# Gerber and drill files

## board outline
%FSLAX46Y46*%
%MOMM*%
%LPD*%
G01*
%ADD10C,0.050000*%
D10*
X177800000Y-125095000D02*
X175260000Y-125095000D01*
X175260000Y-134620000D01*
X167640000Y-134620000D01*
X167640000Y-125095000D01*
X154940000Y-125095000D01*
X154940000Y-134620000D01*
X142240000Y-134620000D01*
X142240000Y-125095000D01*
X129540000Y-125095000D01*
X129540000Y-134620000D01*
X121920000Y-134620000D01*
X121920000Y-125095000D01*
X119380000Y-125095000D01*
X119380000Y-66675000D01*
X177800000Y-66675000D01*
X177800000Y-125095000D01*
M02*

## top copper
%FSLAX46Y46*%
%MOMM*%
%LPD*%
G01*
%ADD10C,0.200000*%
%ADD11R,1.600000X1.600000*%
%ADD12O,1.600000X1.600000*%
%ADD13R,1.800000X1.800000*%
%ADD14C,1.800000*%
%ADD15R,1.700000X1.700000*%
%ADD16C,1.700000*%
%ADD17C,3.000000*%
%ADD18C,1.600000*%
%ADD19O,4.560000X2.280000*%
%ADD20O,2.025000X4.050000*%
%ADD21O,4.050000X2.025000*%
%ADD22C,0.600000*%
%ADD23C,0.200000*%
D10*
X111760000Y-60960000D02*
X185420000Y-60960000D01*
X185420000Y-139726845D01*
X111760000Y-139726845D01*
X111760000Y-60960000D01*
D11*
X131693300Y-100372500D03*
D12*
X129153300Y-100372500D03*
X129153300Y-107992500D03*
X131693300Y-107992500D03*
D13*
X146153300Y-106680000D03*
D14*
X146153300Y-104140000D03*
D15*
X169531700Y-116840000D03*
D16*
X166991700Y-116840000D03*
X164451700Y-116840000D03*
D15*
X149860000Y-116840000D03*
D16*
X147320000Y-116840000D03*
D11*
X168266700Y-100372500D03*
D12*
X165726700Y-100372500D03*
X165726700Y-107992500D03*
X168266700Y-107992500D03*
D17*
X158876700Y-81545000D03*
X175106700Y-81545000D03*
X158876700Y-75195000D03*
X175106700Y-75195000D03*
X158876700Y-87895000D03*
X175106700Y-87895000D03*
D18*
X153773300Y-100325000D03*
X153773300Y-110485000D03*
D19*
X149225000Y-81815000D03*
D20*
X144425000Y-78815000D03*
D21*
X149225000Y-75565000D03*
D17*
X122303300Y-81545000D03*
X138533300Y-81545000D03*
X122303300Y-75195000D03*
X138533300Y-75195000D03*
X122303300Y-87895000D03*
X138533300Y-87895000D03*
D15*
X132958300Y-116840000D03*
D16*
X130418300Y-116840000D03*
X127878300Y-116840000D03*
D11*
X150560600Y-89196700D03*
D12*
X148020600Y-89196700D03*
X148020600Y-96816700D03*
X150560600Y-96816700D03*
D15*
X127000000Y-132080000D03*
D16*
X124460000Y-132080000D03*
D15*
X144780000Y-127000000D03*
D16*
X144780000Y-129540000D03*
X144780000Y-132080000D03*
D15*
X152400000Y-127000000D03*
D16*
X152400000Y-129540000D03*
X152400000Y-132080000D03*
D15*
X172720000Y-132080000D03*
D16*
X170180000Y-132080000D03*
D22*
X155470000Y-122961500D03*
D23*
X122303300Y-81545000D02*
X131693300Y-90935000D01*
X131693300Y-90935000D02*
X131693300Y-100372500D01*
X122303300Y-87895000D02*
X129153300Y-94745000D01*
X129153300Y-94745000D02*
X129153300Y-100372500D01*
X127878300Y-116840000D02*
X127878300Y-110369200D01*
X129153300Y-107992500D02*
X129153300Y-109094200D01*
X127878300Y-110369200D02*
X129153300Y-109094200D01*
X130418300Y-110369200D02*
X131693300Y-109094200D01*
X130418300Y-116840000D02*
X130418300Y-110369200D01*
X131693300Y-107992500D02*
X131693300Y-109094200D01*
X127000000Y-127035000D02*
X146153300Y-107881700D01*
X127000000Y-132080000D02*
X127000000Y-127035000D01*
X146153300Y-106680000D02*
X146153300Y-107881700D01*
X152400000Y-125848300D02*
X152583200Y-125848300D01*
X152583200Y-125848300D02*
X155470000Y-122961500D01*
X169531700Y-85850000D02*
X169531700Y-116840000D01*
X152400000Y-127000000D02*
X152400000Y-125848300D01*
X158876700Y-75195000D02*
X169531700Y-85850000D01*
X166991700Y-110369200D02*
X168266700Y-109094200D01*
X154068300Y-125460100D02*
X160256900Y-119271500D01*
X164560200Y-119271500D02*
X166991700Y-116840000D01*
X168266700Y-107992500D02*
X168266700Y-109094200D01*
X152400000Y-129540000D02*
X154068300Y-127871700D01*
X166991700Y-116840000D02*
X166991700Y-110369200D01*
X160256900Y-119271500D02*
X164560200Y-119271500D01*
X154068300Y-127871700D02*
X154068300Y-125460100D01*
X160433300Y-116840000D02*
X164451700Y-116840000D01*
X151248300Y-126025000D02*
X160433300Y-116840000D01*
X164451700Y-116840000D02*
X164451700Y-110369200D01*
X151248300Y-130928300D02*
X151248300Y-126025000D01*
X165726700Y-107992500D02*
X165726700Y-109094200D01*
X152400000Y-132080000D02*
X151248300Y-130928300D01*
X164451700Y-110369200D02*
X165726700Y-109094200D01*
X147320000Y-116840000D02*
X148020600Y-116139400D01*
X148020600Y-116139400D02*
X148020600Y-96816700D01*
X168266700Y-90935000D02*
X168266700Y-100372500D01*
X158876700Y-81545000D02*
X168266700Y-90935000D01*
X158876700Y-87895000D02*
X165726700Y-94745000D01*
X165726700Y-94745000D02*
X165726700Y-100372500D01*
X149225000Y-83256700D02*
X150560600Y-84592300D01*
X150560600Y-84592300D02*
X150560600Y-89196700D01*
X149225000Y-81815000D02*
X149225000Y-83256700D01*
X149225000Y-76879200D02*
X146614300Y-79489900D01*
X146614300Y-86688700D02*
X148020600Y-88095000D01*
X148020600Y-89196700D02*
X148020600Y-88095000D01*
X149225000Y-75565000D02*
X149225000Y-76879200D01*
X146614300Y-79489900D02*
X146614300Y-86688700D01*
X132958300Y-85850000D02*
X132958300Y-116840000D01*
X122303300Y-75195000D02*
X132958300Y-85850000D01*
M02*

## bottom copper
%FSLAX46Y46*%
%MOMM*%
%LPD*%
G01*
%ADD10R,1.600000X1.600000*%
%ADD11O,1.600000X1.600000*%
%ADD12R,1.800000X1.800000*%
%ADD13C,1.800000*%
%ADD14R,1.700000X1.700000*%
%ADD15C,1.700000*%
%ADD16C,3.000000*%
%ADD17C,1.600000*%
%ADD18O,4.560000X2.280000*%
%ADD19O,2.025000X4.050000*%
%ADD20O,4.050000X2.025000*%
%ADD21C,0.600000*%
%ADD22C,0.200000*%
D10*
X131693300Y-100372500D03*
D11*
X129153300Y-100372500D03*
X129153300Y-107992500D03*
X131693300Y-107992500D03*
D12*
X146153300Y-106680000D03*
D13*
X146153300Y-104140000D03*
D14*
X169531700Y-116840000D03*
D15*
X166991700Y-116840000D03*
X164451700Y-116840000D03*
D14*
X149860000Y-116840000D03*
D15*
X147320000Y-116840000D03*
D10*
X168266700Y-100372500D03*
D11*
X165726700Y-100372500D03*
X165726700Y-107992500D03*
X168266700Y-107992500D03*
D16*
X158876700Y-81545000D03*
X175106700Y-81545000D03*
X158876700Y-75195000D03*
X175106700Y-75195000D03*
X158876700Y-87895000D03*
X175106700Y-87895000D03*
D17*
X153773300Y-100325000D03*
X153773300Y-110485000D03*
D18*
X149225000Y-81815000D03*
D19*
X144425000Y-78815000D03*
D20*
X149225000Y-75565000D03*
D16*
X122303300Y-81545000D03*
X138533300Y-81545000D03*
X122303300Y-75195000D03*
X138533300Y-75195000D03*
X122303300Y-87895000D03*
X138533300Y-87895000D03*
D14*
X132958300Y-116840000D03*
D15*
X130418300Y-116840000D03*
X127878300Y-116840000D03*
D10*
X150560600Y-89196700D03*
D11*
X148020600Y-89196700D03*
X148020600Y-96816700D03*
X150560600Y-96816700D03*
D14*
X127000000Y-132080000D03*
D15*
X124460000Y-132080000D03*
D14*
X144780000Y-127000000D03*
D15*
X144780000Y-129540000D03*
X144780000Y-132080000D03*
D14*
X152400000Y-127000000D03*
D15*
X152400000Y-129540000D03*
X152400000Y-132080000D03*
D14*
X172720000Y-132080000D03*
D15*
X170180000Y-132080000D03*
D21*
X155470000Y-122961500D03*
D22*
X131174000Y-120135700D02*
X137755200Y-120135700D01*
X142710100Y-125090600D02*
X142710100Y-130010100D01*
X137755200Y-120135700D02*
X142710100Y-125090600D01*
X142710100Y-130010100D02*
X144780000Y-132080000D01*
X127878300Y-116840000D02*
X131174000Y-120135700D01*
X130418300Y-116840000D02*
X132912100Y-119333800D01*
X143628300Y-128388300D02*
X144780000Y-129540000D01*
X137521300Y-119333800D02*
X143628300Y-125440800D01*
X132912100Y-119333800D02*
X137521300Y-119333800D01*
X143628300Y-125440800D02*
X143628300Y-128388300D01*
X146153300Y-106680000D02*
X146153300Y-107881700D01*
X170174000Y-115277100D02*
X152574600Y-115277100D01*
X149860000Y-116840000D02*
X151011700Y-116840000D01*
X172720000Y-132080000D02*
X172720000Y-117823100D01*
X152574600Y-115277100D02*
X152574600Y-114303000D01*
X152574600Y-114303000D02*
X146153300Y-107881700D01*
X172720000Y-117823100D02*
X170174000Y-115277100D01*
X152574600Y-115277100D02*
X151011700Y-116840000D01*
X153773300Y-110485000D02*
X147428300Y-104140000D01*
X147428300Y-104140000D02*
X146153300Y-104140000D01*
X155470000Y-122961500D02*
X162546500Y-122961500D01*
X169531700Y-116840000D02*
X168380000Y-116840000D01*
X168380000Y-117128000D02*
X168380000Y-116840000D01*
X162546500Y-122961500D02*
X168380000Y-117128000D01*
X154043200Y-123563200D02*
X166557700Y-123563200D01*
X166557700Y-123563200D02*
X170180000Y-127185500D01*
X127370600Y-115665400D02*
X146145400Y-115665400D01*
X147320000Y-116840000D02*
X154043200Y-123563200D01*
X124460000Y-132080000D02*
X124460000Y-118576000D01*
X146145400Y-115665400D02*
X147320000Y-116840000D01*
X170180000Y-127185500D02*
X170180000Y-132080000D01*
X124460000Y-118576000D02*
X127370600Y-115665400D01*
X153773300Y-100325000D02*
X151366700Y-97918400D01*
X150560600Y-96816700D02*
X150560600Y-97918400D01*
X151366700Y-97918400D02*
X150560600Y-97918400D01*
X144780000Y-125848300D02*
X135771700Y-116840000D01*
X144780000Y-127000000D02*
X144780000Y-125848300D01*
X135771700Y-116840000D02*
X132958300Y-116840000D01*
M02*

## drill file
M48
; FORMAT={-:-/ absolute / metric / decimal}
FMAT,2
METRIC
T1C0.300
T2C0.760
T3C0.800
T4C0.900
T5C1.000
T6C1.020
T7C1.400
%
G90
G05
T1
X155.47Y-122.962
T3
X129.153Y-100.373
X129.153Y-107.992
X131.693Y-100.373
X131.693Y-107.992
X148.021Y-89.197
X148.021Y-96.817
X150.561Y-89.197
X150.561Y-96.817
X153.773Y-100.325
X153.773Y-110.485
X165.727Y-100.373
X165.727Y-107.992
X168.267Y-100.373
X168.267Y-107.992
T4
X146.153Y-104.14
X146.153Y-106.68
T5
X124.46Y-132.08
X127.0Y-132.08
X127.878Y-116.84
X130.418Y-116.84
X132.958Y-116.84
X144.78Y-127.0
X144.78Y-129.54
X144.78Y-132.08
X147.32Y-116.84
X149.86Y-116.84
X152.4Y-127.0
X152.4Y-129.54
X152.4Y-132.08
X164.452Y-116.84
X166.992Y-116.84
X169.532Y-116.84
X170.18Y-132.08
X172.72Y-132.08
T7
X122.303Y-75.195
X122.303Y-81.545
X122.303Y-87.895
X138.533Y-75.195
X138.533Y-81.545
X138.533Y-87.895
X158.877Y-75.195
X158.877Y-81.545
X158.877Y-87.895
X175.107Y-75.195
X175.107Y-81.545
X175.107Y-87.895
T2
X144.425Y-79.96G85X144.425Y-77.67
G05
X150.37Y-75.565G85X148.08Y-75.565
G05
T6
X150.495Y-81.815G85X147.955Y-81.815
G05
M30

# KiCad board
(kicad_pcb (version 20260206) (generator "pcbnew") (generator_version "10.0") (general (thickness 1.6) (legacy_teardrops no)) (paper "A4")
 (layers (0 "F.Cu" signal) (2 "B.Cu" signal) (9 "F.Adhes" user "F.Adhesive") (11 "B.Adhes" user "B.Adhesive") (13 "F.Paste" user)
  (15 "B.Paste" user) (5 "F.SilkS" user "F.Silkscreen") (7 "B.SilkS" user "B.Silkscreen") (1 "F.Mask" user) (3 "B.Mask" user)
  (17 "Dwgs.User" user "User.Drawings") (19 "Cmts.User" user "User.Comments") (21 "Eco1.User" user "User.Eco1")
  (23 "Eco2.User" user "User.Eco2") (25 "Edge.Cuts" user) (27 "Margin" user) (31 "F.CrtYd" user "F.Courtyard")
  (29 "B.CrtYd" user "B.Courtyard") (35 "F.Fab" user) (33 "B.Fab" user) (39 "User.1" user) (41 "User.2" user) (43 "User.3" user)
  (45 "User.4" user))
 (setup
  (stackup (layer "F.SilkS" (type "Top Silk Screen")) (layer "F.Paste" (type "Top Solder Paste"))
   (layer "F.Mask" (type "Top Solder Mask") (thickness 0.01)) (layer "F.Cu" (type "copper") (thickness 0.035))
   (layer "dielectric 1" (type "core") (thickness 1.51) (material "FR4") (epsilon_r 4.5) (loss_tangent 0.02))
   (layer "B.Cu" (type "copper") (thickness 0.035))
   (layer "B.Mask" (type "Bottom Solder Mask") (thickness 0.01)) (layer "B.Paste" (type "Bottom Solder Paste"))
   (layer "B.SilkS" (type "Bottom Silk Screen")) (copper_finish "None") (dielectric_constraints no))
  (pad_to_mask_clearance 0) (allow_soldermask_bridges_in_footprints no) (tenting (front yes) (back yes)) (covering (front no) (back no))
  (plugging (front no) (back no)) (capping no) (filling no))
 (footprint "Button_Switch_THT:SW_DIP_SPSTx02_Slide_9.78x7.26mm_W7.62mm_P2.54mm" (layer "F.Cu") (at 131.6933 100.3725 -90)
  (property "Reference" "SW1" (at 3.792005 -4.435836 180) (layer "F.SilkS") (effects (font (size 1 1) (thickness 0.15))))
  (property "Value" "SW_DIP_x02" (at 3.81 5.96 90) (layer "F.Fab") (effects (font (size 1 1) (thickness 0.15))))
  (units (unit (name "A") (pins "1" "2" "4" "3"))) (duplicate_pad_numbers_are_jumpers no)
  (pad "1" thru_hole rect (at 0 0 270) (size 1.6 1.6) (drill 0.8) (layers "*.Cu" "*.Mask") (remove_unused_layers no)
   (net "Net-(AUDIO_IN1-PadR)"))
  (pad "2" thru_hole oval (at 0 2.54 270) (size 1.6 1.6) (drill 0.8) (layers "*.Cu" "*.Mask") (remove_unused_layers no)
   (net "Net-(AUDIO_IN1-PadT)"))
  (pad "3" thru_hole oval (at 7.62 2.54 270) (size 1.6 1.6) (drill 0.8) (layers "*.Cu" "*.Mask") (remove_unused_layers no)
   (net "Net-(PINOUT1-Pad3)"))
  (pad "4" thru_hole oval (at 7.62 0 270) (size 1.6 1.6) (drill 0.8) (layers "*.Cu" "*.Mask") (remove_unused_layers no)
   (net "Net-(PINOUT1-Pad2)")))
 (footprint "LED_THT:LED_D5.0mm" (layer "F.Cu") (at 146.1533 106.68 90)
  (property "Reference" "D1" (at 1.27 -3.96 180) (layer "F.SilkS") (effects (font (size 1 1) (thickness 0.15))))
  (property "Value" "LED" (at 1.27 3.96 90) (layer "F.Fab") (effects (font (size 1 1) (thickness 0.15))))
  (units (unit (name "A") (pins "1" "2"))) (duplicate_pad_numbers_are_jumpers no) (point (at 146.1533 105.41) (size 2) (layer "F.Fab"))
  (pad "1" thru_hole rect (at 0 0 90) (size 1.8 1.8) (drill 0.9) (layers "*.Cu" "*.Mask") (remove_unused_layers no) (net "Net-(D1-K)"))
  (pad "2" thru_hole circle (at 2.54 0 90) (size 1.8 1.8) (drill 0.9) (layers "*.Cu" "*.Mask") (remove_unused_layers no) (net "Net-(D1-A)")))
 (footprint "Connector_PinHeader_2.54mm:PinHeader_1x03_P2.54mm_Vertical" (layer "F.Cu") (at 169.5317 116.84 -90)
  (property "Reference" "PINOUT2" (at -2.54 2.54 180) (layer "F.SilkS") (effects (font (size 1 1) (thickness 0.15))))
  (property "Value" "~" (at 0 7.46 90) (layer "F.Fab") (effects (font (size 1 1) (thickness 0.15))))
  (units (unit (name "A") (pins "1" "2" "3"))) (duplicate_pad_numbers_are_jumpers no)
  (pad "1" thru_hole rect (at 0 0 270) (size 1.7 1.7) (drill 1) (layers "*.Cu" "*.Mask") (remove_unused_layers no)
   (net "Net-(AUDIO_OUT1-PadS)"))
  (pad "2" thru_hole circle (at 0 2.54 270) (size 1.7 1.7) (drill 1) (layers "*.Cu" "*.Mask") (remove_unused_layers no)
   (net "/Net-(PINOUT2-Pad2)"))
  (pad "3" thru_hole circle (at 0 5.08 270) (size 1.7 1.7) (drill 1) (layers "*.Cu" "*.Mask") (remove_unused_layers no)
   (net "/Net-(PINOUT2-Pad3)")))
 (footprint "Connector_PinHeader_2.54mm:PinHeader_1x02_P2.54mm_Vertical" (layer "F.Cu") (at 149.86 116.84 -90)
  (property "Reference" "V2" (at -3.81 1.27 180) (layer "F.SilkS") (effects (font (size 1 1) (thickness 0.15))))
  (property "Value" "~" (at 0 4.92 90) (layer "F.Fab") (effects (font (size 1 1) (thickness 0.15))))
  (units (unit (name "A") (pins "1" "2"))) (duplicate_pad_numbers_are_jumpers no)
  (pad "1" thru_hole rect (at 0 0 270) (size 1.7 1.7) (drill 1) (layers "*.Cu" "*.Mask") (remove_unused_layers no) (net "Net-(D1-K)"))
  (pad "2" thru_hole circle (at 0 2.54 270) (size 1.7 1.7) (drill 1) (layers "*.Cu" "*.Mask") (remove_unused_layers no)
   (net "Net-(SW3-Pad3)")))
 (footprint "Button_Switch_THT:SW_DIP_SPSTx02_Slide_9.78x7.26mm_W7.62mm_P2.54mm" (layer "F.Cu") (at 168.2667 100.3725 -90)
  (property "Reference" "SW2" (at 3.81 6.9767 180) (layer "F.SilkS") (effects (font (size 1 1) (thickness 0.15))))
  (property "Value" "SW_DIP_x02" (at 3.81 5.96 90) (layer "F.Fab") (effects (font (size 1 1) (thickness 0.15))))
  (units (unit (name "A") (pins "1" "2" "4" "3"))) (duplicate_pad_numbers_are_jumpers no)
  (pad "1" thru_hole rect (at 0 0 270) (size 1.6 1.6) (drill 0.8) (layers "*.Cu" "*.Mask") (remove_unused_layers no)
   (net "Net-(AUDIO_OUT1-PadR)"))
  (pad "2" thru_hole oval (at 0 2.54 270) (size 1.6 1.6) (drill 0.8) (layers "*.Cu" "*.Mask") (remove_unused_layers no)
   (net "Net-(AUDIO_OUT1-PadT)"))
  (pad "3" thru_hole oval (at 7.62 2.54 270) (size 1.6 1.6) (drill 0.8) (layers "*.Cu" "*.Mask") (remove_unused_layers no)
   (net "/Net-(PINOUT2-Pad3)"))
  (pad "4" thru_hole oval (at 7.62 0 270) (size 1.6 1.6) (drill 0.8) (layers "*.Cu" "*.Mask") (remove_unused_layers no)
   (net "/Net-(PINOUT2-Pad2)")))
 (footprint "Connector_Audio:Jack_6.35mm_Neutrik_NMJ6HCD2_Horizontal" (layer "F.Cu") (at 158.8767 87.895 90)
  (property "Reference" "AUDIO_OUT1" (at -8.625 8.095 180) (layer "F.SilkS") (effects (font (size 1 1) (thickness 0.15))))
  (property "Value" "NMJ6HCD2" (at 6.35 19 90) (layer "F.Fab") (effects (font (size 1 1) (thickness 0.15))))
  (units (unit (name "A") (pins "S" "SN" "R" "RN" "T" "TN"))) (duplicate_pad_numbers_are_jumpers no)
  (pad "R" thru_hole circle (at 6.35 0 90) (size 3 3) (drill 1.4) (layers "*.Cu" "*.Mask") (remove_unused_layers no)
   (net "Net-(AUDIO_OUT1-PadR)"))
  (pad "RN" thru_hole circle (at 6.35 16.23 90) (size 3 3) (drill 1.4) (layers "*.Cu" "*.Mask") (remove_unused_layers no)
   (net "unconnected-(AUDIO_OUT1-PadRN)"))
  (pad "S" thru_hole circle (at 12.7 0 90) (size 3 3) (drill 1.4) (layers "*.Cu" "*.Mask") (remove_unused_layers no)
   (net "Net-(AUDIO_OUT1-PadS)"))
  (pad "SN" thru_hole circle (at 12.7 16.23 90) (size 3 3) (drill 1.4) (layers "*.Cu" "*.Mask") (remove_unused_layers no)
   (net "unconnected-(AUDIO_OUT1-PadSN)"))
  (pad "T" thru_hole circle (at 0 0 90) (size 3 3) (drill 1.4) (layers "*.Cu" "*.Mask") (remove_unused_layers no)
   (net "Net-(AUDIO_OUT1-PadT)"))
  (pad "TN" thru_hole circle (at 0 16.23 90) (size 3 3) (drill 1.4) (layers "*.Cu" "*.Mask") (remove_unused_layers no)
   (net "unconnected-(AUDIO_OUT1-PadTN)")))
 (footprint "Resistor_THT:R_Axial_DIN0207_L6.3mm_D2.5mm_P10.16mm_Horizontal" (layer "F.Cu") (at 153.7733 100.325 -90)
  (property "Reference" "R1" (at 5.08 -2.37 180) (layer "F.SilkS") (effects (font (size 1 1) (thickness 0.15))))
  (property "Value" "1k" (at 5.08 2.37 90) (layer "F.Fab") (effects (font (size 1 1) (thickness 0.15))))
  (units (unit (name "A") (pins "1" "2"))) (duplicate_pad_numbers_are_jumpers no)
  (pad "1" thru_hole circle (at 0 0 270) (size 1.6 1.6) (drill 0.8) (layers "*.Cu" "*.Mask") (remove_unused_layers no) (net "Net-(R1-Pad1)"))
  (pad "2" thru_hole circle (at 10.16 0 270) (size 1.6 1.6) (drill 0.8) (layers "*.Cu" "*.Mask") (remove_unused_layers no)
   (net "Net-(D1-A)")))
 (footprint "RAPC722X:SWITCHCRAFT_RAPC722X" (layer "F.Cu") (at 149.225 75.565 180)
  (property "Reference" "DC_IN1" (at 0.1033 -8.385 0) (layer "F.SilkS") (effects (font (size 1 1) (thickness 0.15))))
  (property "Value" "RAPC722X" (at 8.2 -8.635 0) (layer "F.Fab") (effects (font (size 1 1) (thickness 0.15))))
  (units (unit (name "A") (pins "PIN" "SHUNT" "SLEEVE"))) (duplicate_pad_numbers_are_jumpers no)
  (pad "PIN" thru_hole oval (at 0 -6.25 180) (size 4.56 2.28) (drill oval 3.56 1.02) (layers "*.Cu" "*.Mask") (remove_unused_layers no)
   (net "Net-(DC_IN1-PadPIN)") (solder_mask_margin 0.102))
  (pad "SHUNT" thru_hole oval (at 4.8 -3.25 180) (size 2.025 4.05) (drill oval 0.76 3.05) (layers "*.Cu" "*.Mask") (remove_unused_layers no)
   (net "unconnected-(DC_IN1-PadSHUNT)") (solder_mask_margin 0.102))
  (pad "SLEEVE" thru_hole oval (at 0 0 180) (size 4.05 2.025) (drill oval 3.05 0.76) (layers "*.Cu" "*.Mask") (remove_unused_layers no)
   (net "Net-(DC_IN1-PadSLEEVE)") (solder_mask_margin 0.102)))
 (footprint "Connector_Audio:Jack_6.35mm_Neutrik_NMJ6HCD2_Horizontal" (layer "F.Cu") (at 122.3033 87.895 90)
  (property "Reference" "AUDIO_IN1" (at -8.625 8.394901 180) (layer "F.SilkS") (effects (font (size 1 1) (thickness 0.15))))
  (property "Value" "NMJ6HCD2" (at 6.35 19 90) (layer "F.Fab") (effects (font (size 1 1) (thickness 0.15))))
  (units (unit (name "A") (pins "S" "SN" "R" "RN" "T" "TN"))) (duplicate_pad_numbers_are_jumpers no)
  (pad "R" thru_hole circle (at 6.35 0 90) (size 3 3) (drill 1.4) (layers "*.Cu" "*.Mask") (remove_unused_layers no)
   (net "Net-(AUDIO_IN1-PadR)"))
  (pad "RN" thru_hole circle (at 6.35 16.23 90) (size 3 3) (drill 1.4) (layers "*.Cu" "*.Mask") (remove_unused_layers no)
   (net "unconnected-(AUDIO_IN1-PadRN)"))
  (pad "S" thru_hole circle (at 12.7 0 90) (size 3 3) (drill 1.4) (layers "*.Cu" "*.Mask") (remove_unused_layers no)
   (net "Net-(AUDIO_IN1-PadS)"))
  (pad "SN" thru_hole circle (at 12.7 16.23 90) (size 3 3) (drill 1.4) (layers "*.Cu" "*.Mask") (remove_unused_layers no)
   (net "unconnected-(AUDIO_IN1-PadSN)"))
  (pad "T" thru_hole circle (at 0 0 90) (size 3 3) (drill 1.4) (layers "*.Cu" "*.Mask") (remove_unused_layers no)
   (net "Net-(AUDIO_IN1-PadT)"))
  (pad "TN" thru_hole circle (at 0 16.23 90) (size 3 3) (drill 1.4) (layers "*.Cu" "*.Mask") (remove_unused_layers no)
   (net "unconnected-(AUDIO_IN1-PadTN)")))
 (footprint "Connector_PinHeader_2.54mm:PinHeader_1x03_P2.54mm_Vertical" (layer "F.Cu") (at 132.9583 116.84 -90)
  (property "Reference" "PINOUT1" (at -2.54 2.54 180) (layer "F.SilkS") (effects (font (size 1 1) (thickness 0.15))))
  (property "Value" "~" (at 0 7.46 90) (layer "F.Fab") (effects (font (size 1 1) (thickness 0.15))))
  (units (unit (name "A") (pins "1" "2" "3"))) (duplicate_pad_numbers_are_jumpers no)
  (pad "1" thru_hole rect (at 0 0 270) (size 1.7 1.7) (drill 1) (layers "*.Cu" "*.Mask") (remove_unused_layers no)
   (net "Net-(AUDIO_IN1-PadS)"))
  (pad "2" thru_hole circle (at 0 2.54 270) (size 1.7 1.7) (drill 1) (layers "*.Cu" "*.Mask") (remove_unused_layers no)
   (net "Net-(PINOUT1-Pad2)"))
  (pad "3" thru_hole circle (at 0 5.08 270) (size 1.7 1.7) (drill 1) (layers "*.Cu" "*.Mask") (remove_unused_layers no)
   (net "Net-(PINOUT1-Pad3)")))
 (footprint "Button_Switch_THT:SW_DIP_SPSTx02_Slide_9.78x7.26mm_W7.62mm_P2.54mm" (layer "F.Cu") (at 150.5606 89.1967 -90)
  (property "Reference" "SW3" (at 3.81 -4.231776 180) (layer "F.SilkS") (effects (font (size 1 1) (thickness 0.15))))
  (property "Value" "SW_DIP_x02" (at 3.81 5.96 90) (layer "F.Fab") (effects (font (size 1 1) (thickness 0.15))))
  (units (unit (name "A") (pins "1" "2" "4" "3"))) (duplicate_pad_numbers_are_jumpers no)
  (pad "1" thru_hole rect (at 0 0 270) (size 1.6 1.6) (drill 0.8) (layers "*.Cu" "*.Mask") (remove_unused_layers no)
   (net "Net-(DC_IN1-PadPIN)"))
  (pad "2" thru_hole oval (at 0 2.54 270) (size 1.6 1.6) (drill 0.8) (layers "*.Cu" "*.Mask") (remove_unused_layers no)
   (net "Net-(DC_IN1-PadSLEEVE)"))
  (pad "3" thru_hole oval (at 7.62 2.54 270) (size 1.6 1.6) (drill 0.8) (layers "*.Cu" "*.Mask") (remove_unused_layers no)
   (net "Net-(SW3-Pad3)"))
  (pad "4" thru_hole oval (at 7.62 0 270) (size 1.6 1.6) (drill 0.8) (layers "*.Cu" "*.Mask") (remove_unused_layers no)
   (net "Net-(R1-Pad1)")))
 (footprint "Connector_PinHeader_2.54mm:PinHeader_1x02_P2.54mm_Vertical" (layer "B.Cu") (at 127 132.08 90)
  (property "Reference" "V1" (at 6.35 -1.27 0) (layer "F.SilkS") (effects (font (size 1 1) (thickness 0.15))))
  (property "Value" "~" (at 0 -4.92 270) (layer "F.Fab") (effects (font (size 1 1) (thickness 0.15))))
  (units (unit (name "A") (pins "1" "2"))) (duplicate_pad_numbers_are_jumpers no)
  (pad "1" thru_hole rect (at 0 0 90) (size 1.7 1.7) (drill 1) (layers "*.Cu" "*.Mask") (remove_unused_layers no) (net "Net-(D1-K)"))
  (pad "2" thru_hole circle (at 0 -2.54 90) (size 1.7 1.7) (drill 1) (layers "*.Cu" "*.Mask") (remove_unused_layers no)
   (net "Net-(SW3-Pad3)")))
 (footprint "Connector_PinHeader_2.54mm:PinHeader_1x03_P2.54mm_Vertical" (layer "B.Cu") (at 144.78 127 180)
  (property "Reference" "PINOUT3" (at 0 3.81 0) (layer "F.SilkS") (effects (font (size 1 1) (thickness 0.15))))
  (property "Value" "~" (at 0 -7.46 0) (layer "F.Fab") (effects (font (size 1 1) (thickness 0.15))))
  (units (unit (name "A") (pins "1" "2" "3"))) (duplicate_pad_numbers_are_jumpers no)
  (pad "1" thru_hole rect (at 0 0 180) (size 1.7 1.7) (drill 1) (layers "*.Cu" "*.Mask") (remove_unused_layers no)
   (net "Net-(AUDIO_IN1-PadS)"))
  (pad "2" thru_hole circle (at 0 -2.54 180) (size 1.7 1.7) (drill 1) (layers "*.Cu" "*.Mask") (remove_unused_layers no)
   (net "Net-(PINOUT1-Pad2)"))
  (pad "3" thru_hole circle (at 0 -5.08 180) (size 1.7 1.7) (drill 1) (layers "*.Cu" "*.Mask") (remove_unused_layers no)
   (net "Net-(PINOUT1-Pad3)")))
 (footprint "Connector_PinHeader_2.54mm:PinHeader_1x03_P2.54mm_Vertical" (layer "B.Cu") (at 152.4 127 180)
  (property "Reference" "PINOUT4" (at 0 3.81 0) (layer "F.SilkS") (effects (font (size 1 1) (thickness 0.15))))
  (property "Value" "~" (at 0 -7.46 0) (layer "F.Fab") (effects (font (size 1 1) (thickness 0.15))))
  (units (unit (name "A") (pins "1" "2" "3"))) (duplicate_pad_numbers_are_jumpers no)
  (pad "1" thru_hole rect (at 0 0 180) (size 1.7 1.7) (drill 1) (layers "*.Cu" "*.Mask") (remove_unused_layers no)
   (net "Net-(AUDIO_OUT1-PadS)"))
  (pad "2" thru_hole circle (at 0 -2.54 180) (size 1.7 1.7) (drill 1) (layers "*.Cu" "*.Mask") (remove_unused_layers no)
   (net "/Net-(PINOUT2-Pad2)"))
  (pad "3" thru_hole circle (at 0 -5.08 180) (size 1.7 1.7) (drill 1) (layers "*.Cu" "*.Mask") (remove_unused_layers no)
   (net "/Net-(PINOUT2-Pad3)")))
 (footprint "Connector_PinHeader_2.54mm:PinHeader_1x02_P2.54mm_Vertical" (layer "B.Cu") (at 172.72 132.08 90)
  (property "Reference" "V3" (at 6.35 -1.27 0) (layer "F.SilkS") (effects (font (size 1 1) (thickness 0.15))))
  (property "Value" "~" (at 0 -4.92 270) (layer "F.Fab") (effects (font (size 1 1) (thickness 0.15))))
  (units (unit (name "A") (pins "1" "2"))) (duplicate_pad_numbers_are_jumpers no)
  (pad "1" thru_hole rect (at 0 0 90) (size 1.7 1.7) (drill 1) (layers "*.Cu" "*.Mask") (remove_unused_layers no) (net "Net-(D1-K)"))
  (pad "2" thru_hole circle (at 0 -2.54 90) (size 1.7 1.7) (drill 1) (layers "*.Cu" "*.Mask") (remove_unused_layers no)
   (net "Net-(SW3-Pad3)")))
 (gr_rect (start 111.76 60.96) (end 185.42 139.726845) (stroke (width 0.2) (type default)) (fill no) (layer "F.Cu"))
 (gr_poly
  (pts (xy 177.8 125.095) (xy 175.26 125.095) (xy 175.26 134.62) (xy 167.64 134.62) (xy 167.64 125.095) (xy 154.94 125.095)
   (xy 154.94 134.62) (xy 142.24 134.62) (xy 142.24 125.095) (xy 129.54 125.095) (xy 129.54 134.62) (xy 121.92 134.62) (xy 121.92 125.095)
   (xy 119.38 125.095) (xy 119.38 66.675) (xy 177.8 66.675))
  (stroke (width 0.05) (type default)) (fill no) (layer "Edge.Cuts"))
 (segment (start 122.3033 81.545) (end 131.6933 90.935) (width 0.2) (layer "F.Cu") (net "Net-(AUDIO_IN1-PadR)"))
 (segment (start 131.6933 90.935) (end 131.6933 100.3725) (width 0.2) (layer "F.Cu") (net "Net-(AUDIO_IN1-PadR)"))
 (segment (start 122.3033 87.895) (end 129.1533 94.745) (width 0.2) (layer "F.Cu") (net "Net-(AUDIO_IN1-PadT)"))
 (segment (start 129.1533 94.745) (end 129.1533 100.3725) (width 0.2) (layer "F.Cu") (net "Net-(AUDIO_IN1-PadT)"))
 (segment (start 127.8783 116.84) (end 127.8783 110.3692) (width 0.2) (layer "F.Cu") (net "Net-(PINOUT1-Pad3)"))
 (segment (start 129.1533 107.9925) (end 129.1533 109.0942) (width 0.2) (layer "F.Cu") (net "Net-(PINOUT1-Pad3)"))
 (segment (start 127.8783 110.3692) (end 129.1533 109.0942) (width 0.2) (layer "F.Cu") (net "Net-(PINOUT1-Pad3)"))
 (segment (start 131.174 120.1357) (end 137.7552 120.1357) (width 0.2) (layer "B.Cu") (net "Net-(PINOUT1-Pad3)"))
 (segment (start 142.7101 125.0906) (end 142.7101 130.0101) (width 0.2) (layer "B.Cu") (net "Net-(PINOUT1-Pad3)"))
 (segment (start 137.7552 120.1357) (end 142.7101 125.0906) (width 0.2) (layer "B.Cu") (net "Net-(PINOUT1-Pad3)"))
 (segment (start 142.7101 130.0101) (end 144.78 132.08) (width 0.2) (layer "B.Cu") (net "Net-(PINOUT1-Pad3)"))
 (segment (start 127.8783 116.84) (end 131.174 120.1357) (width 0.2) (layer "B.Cu") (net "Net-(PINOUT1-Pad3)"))
 (segment (start 130.4183 110.3692) (end 131.6933 109.0942) (width 0.2) (layer "F.Cu") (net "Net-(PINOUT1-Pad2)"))
 (segment (start 130.4183 116.84) (end 130.4183 110.3692) (width 0.2) (layer "F.Cu") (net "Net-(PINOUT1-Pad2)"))
 (segment (start 131.6933 107.9925) (end 131.6933 109.0942) (width 0.2) (layer "F.Cu") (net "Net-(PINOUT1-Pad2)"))
 (segment (start 130.4183 116.84) (end 132.9121 119.3338) (width 0.2) (layer "B.Cu") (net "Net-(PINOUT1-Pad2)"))
 (segment (start 143.6283 128.3883) (end 144.78 129.54) (width 0.2) (layer "B.Cu") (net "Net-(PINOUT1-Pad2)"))
 (segment (start 137.5213 119.3338) (end 143.6283 125.4408) (width 0.2) (layer "B.Cu") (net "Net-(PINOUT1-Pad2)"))
 (segment (start 132.9121 119.3338) (end 137.5213 119.3338) (width 0.2) (layer "B.Cu") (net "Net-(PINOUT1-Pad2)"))
 (segment (start 143.6283 125.4408) (end 143.6283 128.3883) (width 0.2) (layer "B.Cu") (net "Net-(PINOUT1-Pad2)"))
 (segment (start 127 127.035) (end 146.1533 107.8817) (width 0.2) (layer "F.Cu") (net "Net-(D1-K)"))
 (segment (start 127 132.08) (end 127 127.035) (width 0.2) (layer "F.Cu") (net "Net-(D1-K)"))
 (segment (start 146.1533 106.68) (end 146.1533 107.8817) (width 0.2) (layer "F.Cu") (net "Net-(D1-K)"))
 (segment (start 146.1533 106.68) (end 146.1533 107.8817) (width 0.2) (layer "B.Cu") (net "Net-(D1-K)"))
 (segment (start 170.174 115.2771) (end 152.5746 115.2771) (width 0.2) (layer "B.Cu") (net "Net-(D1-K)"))
 (segment (start 149.86 116.84) (end 151.0117 116.84) (width 0.2) (layer "B.Cu") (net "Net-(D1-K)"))
 (segment (start 172.72 132.08) (end 172.72 117.8231) (width 0.2) (layer "B.Cu") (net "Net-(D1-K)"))
 (segment (start 152.5746 115.2771) (end 152.5746 114.303) (width 0.2) (layer "B.Cu") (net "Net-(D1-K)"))
 (segment (start 152.5746 114.303) (end 146.1533 107.8817) (width 0.2) (layer "B.Cu") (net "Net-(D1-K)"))
 (segment (start 172.72 117.8231) (end 170.174 115.2771) (width 0.2) (layer "B.Cu") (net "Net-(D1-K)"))
 (segment (start 152.5746 115.2771) (end 151.0117 116.84) (width 0.2) (layer "B.Cu") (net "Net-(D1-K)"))
 (segment (start 153.7733 110.485) (end 147.4283 104.14) (width 0.2) (layer "B.Cu") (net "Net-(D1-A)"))
 (segment (start 147.4283 104.14) (end 146.1533 104.14) (width 0.2) (layer "B.Cu") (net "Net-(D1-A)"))
 (segment (start 152.4 125.8483) (end 152.5832 125.8483) (width 0.2) (layer "F.Cu") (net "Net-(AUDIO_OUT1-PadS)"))
 (segment (start 152.5832 125.8483) (end 155.47 122.9615) (width 0.2) (layer "F.Cu") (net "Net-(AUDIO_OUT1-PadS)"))
 (segment (start 169.5317 85.85) (end 169.5317 116.84) (width 0.2) (layer "F.Cu") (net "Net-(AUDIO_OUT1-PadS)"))
 (segment (start 152.4 127) (end 152.4 125.8483) (width 0.2) (layer "F.Cu") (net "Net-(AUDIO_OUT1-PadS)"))
 (segment (start 158.8767 75.195) (end 169.5317 85.85) (width 0.2) (layer "F.Cu") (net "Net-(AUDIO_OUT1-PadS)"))
 (via (at 155.47 122.9615) (size 0.6) (drill 0.3) (layers "F.Cu" "B.Cu") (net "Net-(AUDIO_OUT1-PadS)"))
 (segment (start 155.47 122.9615) (end 162.5465 122.9615) (width 0.2) (layer "B.Cu") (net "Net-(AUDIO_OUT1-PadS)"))
 (segment (start 169.5317 116.84) (end 168.38 116.84) (width 0.2) (layer "B.Cu") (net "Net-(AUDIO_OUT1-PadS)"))
 (segment (start 168.38 117.128) (end 168.38 116.84) (width 0.2) (layer "B.Cu") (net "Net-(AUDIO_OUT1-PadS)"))
 (segment (start 162.5465 122.9615) (end 168.38 117.128) (width 0.2) (layer "B.Cu") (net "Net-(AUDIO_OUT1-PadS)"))
 (segment (start 166.9917 110.3692) (end 168.2667 109.0942) (width 0.2) (layer "F.Cu") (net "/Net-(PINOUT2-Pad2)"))
 (segment (start 154.0683 125.4601) (end 160.2569 119.2715) (width 0.2) (layer "F.Cu") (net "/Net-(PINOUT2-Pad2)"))
 (segment (start 164.5602 119.2715) (end 166.9917 116.84) (width 0.2) (layer "F.Cu") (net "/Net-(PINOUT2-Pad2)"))
 (segment (start 168.2667 107.9925) (end 168.2667 109.0942) (width 0.2) (layer "F.Cu") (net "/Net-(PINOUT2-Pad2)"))
 (segment (start 152.4 129.54) (end 154.0683 127.8717) (width 0.2) (layer "F.Cu") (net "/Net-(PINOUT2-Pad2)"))
 (segment (start 166.9917 116.84) (end 166.9917 110.3692) (width 0.2) (layer "F.Cu") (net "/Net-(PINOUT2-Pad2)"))
 (segment (start 160.2569 119.2715) (end 164.5602 119.2715) (width 0.2) (layer "F.Cu") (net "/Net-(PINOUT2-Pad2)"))
 (segment (start 154.0683 127.8717) (end 154.0683 125.4601) (width 0.2) (layer "F.Cu") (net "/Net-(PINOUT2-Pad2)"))
 (segment (start 160.4333 116.84) (end 164.4517 116.84) (width 0.2) (layer "F.Cu") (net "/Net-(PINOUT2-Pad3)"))
 (segment (start 151.2483 126.025) (end 160.4333 116.84) (width 0.2) (layer "F.Cu") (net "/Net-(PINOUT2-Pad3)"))
 (segment (start 164.4517 116.84) (end 164.4517 110.3692) (width 0.2) (layer "F.Cu") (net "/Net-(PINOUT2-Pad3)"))
 (segment (start 151.2483 130.9283) (end 151.2483 126.025) (width 0.2) (layer "F.Cu") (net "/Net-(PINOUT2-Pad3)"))
 (segment (start 165.7267 107.9925) (end 165.7267 109.0942) (width 0.2) (layer "F.Cu") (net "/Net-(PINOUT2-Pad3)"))
 (segment (start 152.4 132.08) (end 151.2483 130.9283) (width 0.2) (layer "F.Cu") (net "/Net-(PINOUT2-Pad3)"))
 (segment (start 164.4517 110.3692) (end 165.7267 109.0942) (width 0.2) (layer "F.Cu") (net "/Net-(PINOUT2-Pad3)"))
 (segment (start 147.32 116.84) (end 148.0206 116.1394) (width 0.2) (layer "F.Cu") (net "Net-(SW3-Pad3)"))
 (segment (start 148.0206 116.1394) (end 148.0206 96.8167) (width 0.2) (layer "F.Cu") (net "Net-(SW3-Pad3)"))
 (segment (start 154.0432 123.5632) (end 166.5577 123.5632) (width 0.2) (layer "B.Cu") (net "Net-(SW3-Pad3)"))
 (segment (start 166.5577 123.5632) (end 170.18 127.1855) (width 0.2) (layer "B.Cu") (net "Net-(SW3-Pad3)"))
 (segment (start 127.3706 115.6654) (end 146.1454 115.6654) (width 0.2) (layer "B.Cu") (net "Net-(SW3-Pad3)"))
 (segment (start 147.32 116.84) (end 154.0432 123.5632) (width 0.2) (layer "B.Cu") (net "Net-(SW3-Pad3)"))
 (segment (start 124.46 132.08) (end 124.46 118.576) (width 0.2) (layer "B.Cu") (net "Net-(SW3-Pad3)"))
 (segment (start 146.1454 115.6654) (end 147.32 116.84) (width 0.2) (layer "B.Cu") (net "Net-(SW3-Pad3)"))
 (segment (start 170.18 127.1855) (end 170.18 132.08) (width 0.2) (layer "B.Cu") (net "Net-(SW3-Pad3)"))
 (segment (start 124.46 118.576) (end 127.3706 115.6654) (width 0.2) (layer "B.Cu") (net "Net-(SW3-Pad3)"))
 (segment (start 168.2667 90.935) (end 168.2667 100.3725) (width 0.2) (layer "F.Cu") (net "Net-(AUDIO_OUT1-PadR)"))
 (segment (start 158.8767 81.545) (end 168.2667 90.935) (width 0.2) (layer "F.Cu") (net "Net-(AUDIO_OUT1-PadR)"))
 (segment (start 158.8767 87.895) (end 165.7267 94.745) (width 0.2) (layer "F.Cu") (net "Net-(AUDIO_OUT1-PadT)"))
 (segment (start 165.7267 94.745) (end 165.7267 100.3725) (width 0.2) (layer "F.Cu") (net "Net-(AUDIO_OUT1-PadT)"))
 (segment (start 153.7733 100.325) (end 151.3667 97.9184) (width 0.2) (layer "B.Cu") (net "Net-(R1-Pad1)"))
 (segment (start 150.5606 96.8167) (end 150.5606 97.9184) (width 0.2) (layer "B.Cu") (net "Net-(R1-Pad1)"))
 (segment (start 151.3667 97.9184) (end 150.5606 97.9184) (width 0.2) (layer "B.Cu") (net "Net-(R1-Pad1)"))
 (segment (start 149.225 83.2567) (end 150.5606 84.5923) (width 0.2) (layer "F.Cu") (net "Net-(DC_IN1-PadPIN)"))
 (segment (start 150.5606 84.5923) (end 150.5606 89.1967) (width 0.2) (layer "F.Cu") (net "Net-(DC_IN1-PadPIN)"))
 (segment (start 149.225 81.815) (end 149.225 83.2567) (width 0.2) (layer "F.Cu") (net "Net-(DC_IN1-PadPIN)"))
 (segment (start 149.225 76.8792) (end 146.6143 79.4899) (width 0.2) (layer "F.Cu") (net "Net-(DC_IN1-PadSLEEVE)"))
 (segment (start 146.6143 86.6887) (end 148.0206 88.095) (width 0.2) (layer "F.Cu") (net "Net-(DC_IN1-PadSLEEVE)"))
 (segment (start 148.0206 89.1967) (end 148.0206 88.095) (width 0.2) (layer "F.Cu") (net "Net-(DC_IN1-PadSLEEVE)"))
 (segment (start 149.225 75.565) (end 149.225 76.8792) (width 0.2) (layer "F.Cu") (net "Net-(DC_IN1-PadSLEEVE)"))
 (segment (start 146.6143 79.4899) (end 146.6143 86.6887) (width 0.2) (layer "F.Cu") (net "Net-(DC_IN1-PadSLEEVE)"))
 (segment (start 132.9583 85.85) (end 132.9583 116.84) (width 0.2) (layer "F.Cu") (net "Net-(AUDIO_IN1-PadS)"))
 (segment (start 122.3033 75.195) (end 132.9583 85.85) (width 0.2) (layer "F.Cu") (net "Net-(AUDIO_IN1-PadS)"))
 (segment (start 144.78 125.8483) (end 135.7717 116.84) (width 0.2) (layer "B.Cu") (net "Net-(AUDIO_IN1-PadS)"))
 (segment (start 144.78 127) (end 144.78 125.8483) (width 0.2) (layer "B.Cu") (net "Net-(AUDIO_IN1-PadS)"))
 (segment (start 135.7717 116.84) (end 132.9583 116.84) (width 0.2) (layer "B.Cu") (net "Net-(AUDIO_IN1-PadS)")))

